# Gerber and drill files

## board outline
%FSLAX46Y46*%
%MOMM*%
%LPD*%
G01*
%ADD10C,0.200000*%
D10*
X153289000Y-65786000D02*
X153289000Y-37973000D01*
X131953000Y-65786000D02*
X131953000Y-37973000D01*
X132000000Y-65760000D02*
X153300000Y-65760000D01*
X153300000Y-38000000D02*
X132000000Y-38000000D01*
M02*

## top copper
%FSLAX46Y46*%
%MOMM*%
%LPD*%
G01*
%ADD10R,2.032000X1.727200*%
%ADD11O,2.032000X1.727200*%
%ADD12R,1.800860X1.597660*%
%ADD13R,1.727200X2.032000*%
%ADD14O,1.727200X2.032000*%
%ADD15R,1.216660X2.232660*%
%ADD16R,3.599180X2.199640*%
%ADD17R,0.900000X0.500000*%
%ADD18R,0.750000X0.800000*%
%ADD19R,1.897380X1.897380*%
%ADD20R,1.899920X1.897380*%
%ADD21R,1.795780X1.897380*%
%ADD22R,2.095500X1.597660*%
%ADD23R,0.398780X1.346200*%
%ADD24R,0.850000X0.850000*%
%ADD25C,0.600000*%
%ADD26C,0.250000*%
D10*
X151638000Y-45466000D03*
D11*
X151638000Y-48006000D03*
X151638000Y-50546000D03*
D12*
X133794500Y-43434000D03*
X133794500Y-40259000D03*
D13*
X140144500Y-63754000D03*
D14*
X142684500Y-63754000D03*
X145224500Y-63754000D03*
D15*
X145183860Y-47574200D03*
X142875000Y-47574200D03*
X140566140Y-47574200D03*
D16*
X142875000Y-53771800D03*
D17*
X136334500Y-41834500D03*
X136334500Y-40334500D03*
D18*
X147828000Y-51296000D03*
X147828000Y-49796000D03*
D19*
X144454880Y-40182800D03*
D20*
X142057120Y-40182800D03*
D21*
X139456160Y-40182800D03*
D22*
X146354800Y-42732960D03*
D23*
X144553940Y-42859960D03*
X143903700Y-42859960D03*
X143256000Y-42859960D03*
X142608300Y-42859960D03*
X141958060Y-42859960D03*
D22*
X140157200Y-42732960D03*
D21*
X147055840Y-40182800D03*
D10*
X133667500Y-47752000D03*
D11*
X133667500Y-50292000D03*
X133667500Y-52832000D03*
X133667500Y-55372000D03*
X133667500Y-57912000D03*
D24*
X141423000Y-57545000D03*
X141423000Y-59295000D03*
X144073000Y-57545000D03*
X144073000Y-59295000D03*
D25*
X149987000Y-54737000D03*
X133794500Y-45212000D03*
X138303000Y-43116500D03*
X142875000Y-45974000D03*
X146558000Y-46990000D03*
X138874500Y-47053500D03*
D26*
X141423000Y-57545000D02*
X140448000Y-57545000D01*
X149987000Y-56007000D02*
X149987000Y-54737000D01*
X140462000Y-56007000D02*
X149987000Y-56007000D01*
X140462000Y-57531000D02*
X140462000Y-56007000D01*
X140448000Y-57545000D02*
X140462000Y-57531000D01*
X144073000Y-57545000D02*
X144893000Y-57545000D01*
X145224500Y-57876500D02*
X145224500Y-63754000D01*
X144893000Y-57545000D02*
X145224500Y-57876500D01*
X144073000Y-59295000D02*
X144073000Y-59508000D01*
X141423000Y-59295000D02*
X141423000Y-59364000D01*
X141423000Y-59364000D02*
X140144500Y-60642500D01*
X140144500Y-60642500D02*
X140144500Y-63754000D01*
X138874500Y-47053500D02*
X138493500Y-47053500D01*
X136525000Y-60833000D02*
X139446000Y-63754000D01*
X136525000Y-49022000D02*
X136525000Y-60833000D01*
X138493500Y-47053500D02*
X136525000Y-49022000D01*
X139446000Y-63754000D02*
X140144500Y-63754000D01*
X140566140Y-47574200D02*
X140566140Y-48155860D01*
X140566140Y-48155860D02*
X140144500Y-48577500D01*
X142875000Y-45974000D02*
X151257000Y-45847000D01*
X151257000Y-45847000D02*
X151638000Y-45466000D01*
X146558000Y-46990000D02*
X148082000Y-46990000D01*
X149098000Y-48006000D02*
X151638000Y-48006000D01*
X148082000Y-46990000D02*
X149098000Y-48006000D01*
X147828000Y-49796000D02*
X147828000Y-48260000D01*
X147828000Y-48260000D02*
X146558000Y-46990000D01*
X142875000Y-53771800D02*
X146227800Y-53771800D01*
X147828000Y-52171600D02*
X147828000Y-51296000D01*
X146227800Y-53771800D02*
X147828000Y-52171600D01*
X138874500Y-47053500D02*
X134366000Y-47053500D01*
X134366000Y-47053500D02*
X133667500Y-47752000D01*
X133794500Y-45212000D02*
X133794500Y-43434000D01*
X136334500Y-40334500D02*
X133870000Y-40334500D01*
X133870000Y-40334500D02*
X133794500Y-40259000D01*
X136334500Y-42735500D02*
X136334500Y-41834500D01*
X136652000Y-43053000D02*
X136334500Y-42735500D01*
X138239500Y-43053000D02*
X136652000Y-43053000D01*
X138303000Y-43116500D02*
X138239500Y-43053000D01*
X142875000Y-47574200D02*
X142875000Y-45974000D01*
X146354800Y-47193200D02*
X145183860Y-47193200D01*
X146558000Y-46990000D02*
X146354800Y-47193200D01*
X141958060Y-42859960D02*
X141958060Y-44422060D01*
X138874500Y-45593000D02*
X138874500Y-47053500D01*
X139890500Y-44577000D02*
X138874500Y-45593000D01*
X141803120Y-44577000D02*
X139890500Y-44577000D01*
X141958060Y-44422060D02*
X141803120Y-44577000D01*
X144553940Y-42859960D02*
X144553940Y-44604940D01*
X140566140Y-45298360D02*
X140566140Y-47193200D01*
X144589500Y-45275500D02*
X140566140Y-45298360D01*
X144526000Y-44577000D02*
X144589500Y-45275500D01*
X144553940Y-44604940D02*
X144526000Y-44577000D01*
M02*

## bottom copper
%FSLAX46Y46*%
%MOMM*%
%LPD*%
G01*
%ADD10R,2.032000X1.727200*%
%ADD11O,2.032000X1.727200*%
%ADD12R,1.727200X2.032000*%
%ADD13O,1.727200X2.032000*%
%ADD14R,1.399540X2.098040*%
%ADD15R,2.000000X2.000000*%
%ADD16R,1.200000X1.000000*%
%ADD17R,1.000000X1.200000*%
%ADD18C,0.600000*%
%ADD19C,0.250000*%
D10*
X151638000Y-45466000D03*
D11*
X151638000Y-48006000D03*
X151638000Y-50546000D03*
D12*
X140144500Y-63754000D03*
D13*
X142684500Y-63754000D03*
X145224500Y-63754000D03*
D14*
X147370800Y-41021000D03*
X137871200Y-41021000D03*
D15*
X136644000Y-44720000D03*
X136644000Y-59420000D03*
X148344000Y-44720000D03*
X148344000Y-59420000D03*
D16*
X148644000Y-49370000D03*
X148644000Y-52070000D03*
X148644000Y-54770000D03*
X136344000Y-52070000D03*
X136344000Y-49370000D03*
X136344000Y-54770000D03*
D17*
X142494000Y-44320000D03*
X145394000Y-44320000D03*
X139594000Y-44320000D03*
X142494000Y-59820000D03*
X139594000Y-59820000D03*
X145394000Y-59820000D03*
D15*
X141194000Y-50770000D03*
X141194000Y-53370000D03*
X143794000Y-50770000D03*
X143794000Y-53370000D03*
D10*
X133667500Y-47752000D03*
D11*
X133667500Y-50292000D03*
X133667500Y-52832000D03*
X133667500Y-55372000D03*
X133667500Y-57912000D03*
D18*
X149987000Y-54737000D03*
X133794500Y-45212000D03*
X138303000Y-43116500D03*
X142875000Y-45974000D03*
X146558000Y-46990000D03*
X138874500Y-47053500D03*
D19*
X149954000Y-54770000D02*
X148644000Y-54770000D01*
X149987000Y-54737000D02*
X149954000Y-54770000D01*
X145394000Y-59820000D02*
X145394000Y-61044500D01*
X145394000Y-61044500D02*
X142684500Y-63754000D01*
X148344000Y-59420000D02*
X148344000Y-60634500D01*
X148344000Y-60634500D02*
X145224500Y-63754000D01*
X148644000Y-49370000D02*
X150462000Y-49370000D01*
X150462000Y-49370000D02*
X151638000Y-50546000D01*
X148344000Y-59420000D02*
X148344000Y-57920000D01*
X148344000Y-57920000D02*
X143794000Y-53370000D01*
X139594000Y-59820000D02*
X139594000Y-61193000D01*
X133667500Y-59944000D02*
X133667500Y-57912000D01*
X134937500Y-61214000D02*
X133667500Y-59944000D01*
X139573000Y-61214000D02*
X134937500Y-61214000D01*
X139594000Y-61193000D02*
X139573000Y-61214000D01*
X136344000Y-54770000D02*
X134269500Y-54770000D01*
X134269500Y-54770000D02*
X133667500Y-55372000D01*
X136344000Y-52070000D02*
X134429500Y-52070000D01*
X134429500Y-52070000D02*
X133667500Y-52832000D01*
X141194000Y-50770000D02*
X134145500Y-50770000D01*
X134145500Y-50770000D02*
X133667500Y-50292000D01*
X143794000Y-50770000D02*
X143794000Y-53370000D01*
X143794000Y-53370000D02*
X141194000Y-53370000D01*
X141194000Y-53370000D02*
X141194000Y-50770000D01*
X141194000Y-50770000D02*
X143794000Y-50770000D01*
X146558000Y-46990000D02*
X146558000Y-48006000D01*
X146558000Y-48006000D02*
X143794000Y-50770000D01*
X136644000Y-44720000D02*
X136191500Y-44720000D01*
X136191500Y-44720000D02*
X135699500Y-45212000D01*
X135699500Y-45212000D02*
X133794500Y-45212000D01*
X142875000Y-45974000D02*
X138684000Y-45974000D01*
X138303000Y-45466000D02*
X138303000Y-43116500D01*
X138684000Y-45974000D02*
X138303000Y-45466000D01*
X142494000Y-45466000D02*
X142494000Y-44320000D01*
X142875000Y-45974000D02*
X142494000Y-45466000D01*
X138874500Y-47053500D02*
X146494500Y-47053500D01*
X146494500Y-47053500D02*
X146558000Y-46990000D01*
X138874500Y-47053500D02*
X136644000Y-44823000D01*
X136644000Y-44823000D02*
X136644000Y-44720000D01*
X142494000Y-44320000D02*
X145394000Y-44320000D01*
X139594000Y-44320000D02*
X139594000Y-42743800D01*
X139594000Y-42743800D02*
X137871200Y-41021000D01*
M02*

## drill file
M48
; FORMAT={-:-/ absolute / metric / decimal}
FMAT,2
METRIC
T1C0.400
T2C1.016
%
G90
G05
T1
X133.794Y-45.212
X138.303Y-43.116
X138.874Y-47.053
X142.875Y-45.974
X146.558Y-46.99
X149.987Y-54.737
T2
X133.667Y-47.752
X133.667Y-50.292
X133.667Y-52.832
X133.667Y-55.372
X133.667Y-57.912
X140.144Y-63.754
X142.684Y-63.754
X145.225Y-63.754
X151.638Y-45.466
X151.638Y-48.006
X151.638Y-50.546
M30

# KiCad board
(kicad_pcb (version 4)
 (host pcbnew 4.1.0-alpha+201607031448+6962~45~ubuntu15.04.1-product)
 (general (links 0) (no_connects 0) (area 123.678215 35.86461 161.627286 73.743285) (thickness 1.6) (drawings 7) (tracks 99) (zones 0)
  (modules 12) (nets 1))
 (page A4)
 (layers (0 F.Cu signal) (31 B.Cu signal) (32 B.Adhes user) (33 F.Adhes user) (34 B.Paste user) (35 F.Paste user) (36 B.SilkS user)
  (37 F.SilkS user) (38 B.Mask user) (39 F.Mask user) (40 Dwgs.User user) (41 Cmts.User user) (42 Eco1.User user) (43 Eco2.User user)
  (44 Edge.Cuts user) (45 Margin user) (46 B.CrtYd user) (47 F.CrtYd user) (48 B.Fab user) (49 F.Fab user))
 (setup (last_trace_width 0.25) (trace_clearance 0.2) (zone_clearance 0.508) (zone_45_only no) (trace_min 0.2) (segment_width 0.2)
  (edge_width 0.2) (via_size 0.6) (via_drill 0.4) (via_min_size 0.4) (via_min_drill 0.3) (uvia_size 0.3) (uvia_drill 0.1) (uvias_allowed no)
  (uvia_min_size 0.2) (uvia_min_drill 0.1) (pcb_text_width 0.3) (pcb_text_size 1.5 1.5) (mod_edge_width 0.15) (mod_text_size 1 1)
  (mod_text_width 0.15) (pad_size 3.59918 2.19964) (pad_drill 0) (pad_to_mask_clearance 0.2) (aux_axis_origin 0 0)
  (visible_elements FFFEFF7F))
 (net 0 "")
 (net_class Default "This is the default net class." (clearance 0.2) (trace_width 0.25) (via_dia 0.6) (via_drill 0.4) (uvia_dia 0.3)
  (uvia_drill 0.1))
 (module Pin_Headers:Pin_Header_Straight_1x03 (layer F.Cu) (at 151.638 45.466)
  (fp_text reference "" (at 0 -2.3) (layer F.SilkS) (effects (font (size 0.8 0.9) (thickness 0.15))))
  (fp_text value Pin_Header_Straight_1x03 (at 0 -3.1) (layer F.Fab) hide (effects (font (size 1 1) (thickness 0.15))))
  (pad 1 thru_hole rect (at 0 0) (size 2.032 1.7272) (drill 1.016) (layers *.Cu *.Mask F.SilkS))
  (pad 2 thru_hole oval (at 0 2.54) (size 2.032 1.7272) (drill 1.016) (layers *.Cu *.Mask F.SilkS))
  (pad 3 thru_hole oval (at 0 5.08) (size 2.032 1.7272) (drill 1.016) (layers *.Cu *.Mask F.SilkS)))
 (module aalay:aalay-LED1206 (layer F.Cu) (at 133.7945 41.8465 90)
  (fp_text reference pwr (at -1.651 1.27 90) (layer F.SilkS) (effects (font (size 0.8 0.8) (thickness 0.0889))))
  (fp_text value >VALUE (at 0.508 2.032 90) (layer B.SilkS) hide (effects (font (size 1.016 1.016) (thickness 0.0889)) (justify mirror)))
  (pad A smd rect (at -1.5875 0 90) (size 1.59766 1.80086) (layers F.Cu F.Paste F.Mask))
  (pad K smd rect (at 1.5875 0 90) (size 1.59766 1.80086) (layers F.Cu F.Paste F.Mask)))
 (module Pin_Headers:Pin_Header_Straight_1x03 (layer F.Cu) (at 140.1445 63.754 90)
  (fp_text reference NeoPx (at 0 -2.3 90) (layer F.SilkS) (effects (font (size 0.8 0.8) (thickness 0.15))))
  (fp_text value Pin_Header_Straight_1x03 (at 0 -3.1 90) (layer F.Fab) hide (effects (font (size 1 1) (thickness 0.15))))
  (pad 1 thru_hole rect (at 0 0 90) (size 2.032 1.7272) (drill 1.016) (layers *.Cu *.Mask F.SilkS))
  (pad 2 thru_hole oval (at 0 2.54 90) (size 2.032 1.7272) (drill 1.016) (layers *.Cu *.Mask F.SilkS))
  (pad 3 thru_hole oval (at 0 5.08 90) (size 2.032 1.7272) (drill 1.016) (layers *.Cu *.Mask F.SilkS)))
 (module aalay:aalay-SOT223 (layer F.Cu) (at 142.875 50.673 180)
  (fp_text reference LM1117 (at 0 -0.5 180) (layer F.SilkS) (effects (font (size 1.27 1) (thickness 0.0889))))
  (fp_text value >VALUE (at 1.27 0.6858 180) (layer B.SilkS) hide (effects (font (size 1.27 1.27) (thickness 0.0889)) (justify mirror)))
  (pad GND smd rect (at -2.30886 3.0988 180) (size 1.21666 2.23266) (layers F.Cu F.Paste F.Mask))
  (pad OUT smd rect (at 0 3.0988 180) (size 1.21666 2.23266) (layers F.Cu F.Paste F.Mask))
  (pad IN smd rect (at 2.30886 3.0988 180) (size 1.21666 2.23266) (layers F.Cu F.Paste F.Mask))
  (pad OUT smd rect (at 0 -3.0988 180) (size 3.59918 2.19964) (layers F.Cu F.Paste F.Mask)))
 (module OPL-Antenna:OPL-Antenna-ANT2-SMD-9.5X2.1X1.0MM (layer B.Cu) (at 142.621 41.021 180)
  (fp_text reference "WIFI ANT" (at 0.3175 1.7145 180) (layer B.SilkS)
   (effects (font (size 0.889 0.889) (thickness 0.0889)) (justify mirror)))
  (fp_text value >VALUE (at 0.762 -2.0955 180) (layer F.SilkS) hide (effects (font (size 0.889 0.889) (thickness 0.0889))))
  (pad 1 smd rect (at -4.7498 0 180) (size 1.39954 2.09804) (layers B.Cu B.Paste B.Mask))
  (pad 2 smd rect (at 4.7498 0 180) (size 1.39954 2.09804) (layers B.Cu B.Paste B.Mask)))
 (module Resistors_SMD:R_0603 (layer F.Cu) (at 136.3345 41.0845 90)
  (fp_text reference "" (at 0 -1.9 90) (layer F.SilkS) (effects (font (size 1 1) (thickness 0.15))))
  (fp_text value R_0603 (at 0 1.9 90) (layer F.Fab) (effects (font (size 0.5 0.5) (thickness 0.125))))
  (pad 1 smd rect (at -0.75 0 90) (size 0.5 0.9) (layers F.Cu F.Paste F.Mask))
  (pad 2 smd rect (at 0.75 0 90) (size 0.5 0.9) (layers F.Cu F.Paste F.Mask)))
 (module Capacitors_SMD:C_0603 (layer F.Cu) (at 147.828 50.546 90)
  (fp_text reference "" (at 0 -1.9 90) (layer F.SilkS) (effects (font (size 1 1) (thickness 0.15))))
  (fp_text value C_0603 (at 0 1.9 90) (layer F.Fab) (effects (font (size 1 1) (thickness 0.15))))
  (pad 1 smd rect (at -0.75 0 90) (size 0.8 0.75) (layers F.Cu F.Paste F.Mask))
  (pad 2 smd rect (at 0.75 0 90) (size 0.8 0.75) (layers F.Cu F.Paste F.Mask)))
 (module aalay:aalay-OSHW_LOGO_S (layer F.Cu) (at 150.622 39.878)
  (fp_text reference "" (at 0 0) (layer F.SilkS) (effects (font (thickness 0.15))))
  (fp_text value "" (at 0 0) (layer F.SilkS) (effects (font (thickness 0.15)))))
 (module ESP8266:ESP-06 (layer B.Cu) (at 142.494 52.07 270)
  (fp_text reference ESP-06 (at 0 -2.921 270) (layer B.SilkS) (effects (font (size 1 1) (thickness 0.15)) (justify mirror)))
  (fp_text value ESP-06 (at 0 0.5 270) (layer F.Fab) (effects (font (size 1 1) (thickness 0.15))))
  (pad GND smd rect (at -7.35 5.85 270) (size 2 2) (layers B.Cu B.Paste B.Mask))
  (pad GP5 smd rect (at 7.35 5.85 270) (size 2 2) (layers B.Cu B.Paste B.Mask))
  (pad GP16 smd rect (at -7.35 -5.85 270) (size 2 2) (layers B.Cu B.Paste B.Mask))
  (pad GP15 smd rect (at 7.35 -5.85 270) (size 2 2) (layers B.Cu B.Paste B.Mask))
  (pad GP14 smd rect (at -2.7 -6.15 270) (size 1 1.2) (layers B.Cu B.Paste B.Mask))
  (pad GP12 smd rect (at 0 -6.15 270) (size 1 1.2) (layers B.Cu B.Paste B.Mask))
  (pad GP13 smd rect (at 2.7 -6.15 270) (size 1 1.2) (layers B.Cu B.Paste B.Mask))
  (pad TX smd rect (at 0 6.15 270) (size 1 1.2) (layers B.Cu B.Paste B.Mask))
  (pad RST smd rect (at -2.7 6.15 270) (size 1 1.2) (layers B.Cu B.Paste B.Mask))
  (pad RX smd rect (at 2.7 6.15 270) (size 1 1.2) (layers B.Cu B.Paste B.Mask))
  (pad 3.3 smd rect (at -7.75 0 270) (size 1.2 1) (layers B.Cu B.Paste B.Mask))
  (pad CHPD smd rect (at -7.75 -2.9 270) (size 1.2 1) (layers B.Cu B.Paste B.Mask))
  (pad ANT smd rect (at -7.75 2.9 270) (size 1.2 1) (layers B.Cu B.Paste B.Mask))
  (pad GP2 smd rect (at 7.75 0 270) (size 1.2 1) (layers B.Cu B.Paste B.Mask))
  (pad GP0 smd rect (at 7.75 2.9 270) (size 1.2 1) (layers B.Cu B.Paste B.Mask))
  (pad GP4 smd rect (at 7.75 -2.9 270) (size 1.2 1) (layers B.Cu B.Paste B.Mask))
  (pad GND smd rect (at -1.3 1.3 270) (size 2 2) (layers B.Cu B.Paste B.Mask))
  (pad GND smd rect (at 1.3 1.3 270) (size 2 2) (layers B.Cu B.Paste B.Mask))
  (pad GND smd rect (at -1.3 -1.3 270) (size 2 2) (layers B.Cu B.Paste B.Mask))
  (pad GND smd rect (at 1.3 -1.3 270) (size 2 2) (layers B.Cu B.Paste B.Mask)))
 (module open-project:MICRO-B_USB (layer F.Cu) (at 143.256 38.735 180)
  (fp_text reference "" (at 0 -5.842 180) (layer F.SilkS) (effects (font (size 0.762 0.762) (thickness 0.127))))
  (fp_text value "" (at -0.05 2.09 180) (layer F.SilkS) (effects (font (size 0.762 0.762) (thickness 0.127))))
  (pad "" smd rect (at -1.19888 -1.4478 180) (size 1.89738 1.89738) (layers F.Cu F.Paste F.Mask))
  (pad "" smd rect (at 1.19888 -1.4478 180) (size 1.89992 1.89738) (layers F.Cu F.Paste F.Mask))
  (pad "" smd rect (at 3.79984 -1.4478 180) (size 1.79578 1.89738) (layers F.Cu F.Paste F.Mask))
  (pad "" smd rect (at -3.0988 -3.99796 180) (size 2.0955 1.59766) (layers F.Cu F.Paste F.Mask))
  (pad 1 smd rect (at -1.29794 -4.12496 180) (size 0.39878 1.3462) (layers F.Cu F.Paste F.Mask) (clearance 0.2032))
  (pad 2 smd rect (at -0.6477 -4.12496 180) (size 0.39878 1.3462) (layers F.Cu F.Paste F.Mask) (clearance 0.2032))
  (pad 3 smd rect (at 0 -4.12496 180) (size 0.39878 1.3462) (layers F.Cu F.Paste F.Mask) (clearance 0.2032))
  (pad 4 smd rect (at 0.6477 -4.12496 180) (size 0.39878 1.3462) (layers F.Cu F.Paste F.Mask) (clearance 0.2032))
  (pad 5 smd rect (at 1.29794 -4.12496 180) (size 0.39878 1.3462) (layers F.Cu F.Paste F.Mask) (clearance 0.2032))
  (pad "" smd rect (at 3.0988 -3.99796 180) (size 2.0955 1.59766) (layers F.Cu F.Paste F.Mask))
  (pad "" smd rect (at -3.79984 -1.4478 180) (size 1.79578 1.89738) (layers F.Cu F.Paste F.Mask)))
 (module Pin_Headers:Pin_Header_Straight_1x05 (layer F.Cu) (at 133.6675 47.752)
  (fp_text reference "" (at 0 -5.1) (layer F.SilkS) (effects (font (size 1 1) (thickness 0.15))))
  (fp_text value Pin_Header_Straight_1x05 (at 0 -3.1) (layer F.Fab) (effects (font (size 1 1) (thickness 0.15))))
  (pad 1 thru_hole rect (at 0 0) (size 2.032 1.7272) (drill 1.016) (layers *.Cu *.Mask F.SilkS))
  (pad 2 thru_hole oval (at 0 2.54) (size 2.032 1.7272) (drill 1.016) (layers *.Cu *.Mask F.SilkS))
  (pad 3 thru_hole oval (at 0 5.08) (size 2.032 1.7272) (drill 1.016) (layers *.Cu *.Mask F.SilkS))
  (pad 4 thru_hole oval (at 0 7.62) (size 2.032 1.7272) (drill 1.016) (layers *.Cu *.Mask F.SilkS))
  (pad 5 thru_hole oval (at 0 10.16) (size 2.032 1.7272) (drill 1.016) (layers *.Cu *.Mask F.SilkS)))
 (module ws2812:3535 (layer F.Cu) (at 142.748 58.42 180)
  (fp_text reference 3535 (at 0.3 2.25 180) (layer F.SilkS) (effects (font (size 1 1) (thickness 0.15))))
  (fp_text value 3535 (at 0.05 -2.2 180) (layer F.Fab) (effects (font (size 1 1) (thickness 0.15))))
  (pad IN smd rect (at 1.325 0.875 180) (size 0.85 0.85) (layers F.Cu F.Paste F.Mask))
  (pad VDD smd rect (at 1.325 -0.875 180) (size 0.85 0.85) (layers F.Cu F.Paste F.Mask))
  (pad VSS smd rect (at -1.325 0.875 180) (size 0.85 0.85) (layers F.Cu F.Paste F.Mask))
  (pad OUT smd rect (at -1.325 -0.875 180) (size 0.85 0.85) (layers F.Cu F.Paste F.Mask)))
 (gr_line (start 153.289 65.786) (end 153.289 37.973) (angle 90) (layer Edge.Cuts) (width 0.2))
 (gr_line (start 131.953 65.786) (end 131.953 37.973) (angle 90) (layer Edge.Cuts) (width 0.2))
 (gr_line (start 132 65.76) (end 153.3 65.76) (angle 90) (layer Edge.Cuts) (width 0.2))
 (gr_line (start 153.3 38) (end 132 38) (angle 90) (layer Edge.Cuts) (width 0.2))
 (segment (start 141.423 57.545) (end 140.448 57.545) (width 0.25) (layer F.Cu) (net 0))
 (segment (start 149.954 54.77) (end 148.644 54.77) (width 0.25) (layer B.Cu) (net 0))
 (segment (start 149.987 54.737) (end 149.954 54.77) (width 0.25) (layer B.Cu) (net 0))
 (via (at 149.987 54.737) (size 0.6) (drill 0.4) (layers F.Cu B.Cu) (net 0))
 (segment (start 149.987 56.007) (end 149.987 54.737) (width 0.25) (layer F.Cu) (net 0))
 (segment (start 140.462 56.007) (end 149.987 56.007) (width 0.25) (layer F.Cu) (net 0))
 (segment (start 140.462 57.531) (end 140.462 56.007) (width 0.25) (layer F.Cu) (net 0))
 (segment (start 140.448 57.545) (end 140.462 57.531) (width 0.25) (layer F.Cu) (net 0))
 (segment (start 144.073 57.545) (end 144.893 57.545) (width 0.25) (layer F.Cu) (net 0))
 (segment (start 145.2245 57.8765) (end 145.2245 63.754) (width 0.25) (layer F.Cu) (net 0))
 (segment (start 144.893 57.545) (end 145.2245 57.8765) (width 0.25) (layer F.Cu) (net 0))
 (segment (start 144.073 59.295) (end 144.073 59.508) (width 0.25) (layer F.Cu) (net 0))
 (segment (start 141.423 59.295) (end 141.423 59.364) (width 0.25) (layer F.Cu) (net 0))
 (segment (start 141.423 59.364) (end 140.1445 60.6425) (width 0.25) (layer F.Cu) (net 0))
 (segment (start 140.1445 60.6425) (end 140.1445 63.754) (width 0.25) (layer F.Cu) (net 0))
 (segment (start 138.8745 47.0535) (end 138.4935 47.0535) (width 0.25) (layer F.Cu) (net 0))
 (segment (start 136.525 60.833) (end 139.446 63.754) (width 0.25) (layer F.Cu) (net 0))
 (segment (start 136.525 49.022) (end 136.525 60.833) (width 0.25) (layer F.Cu) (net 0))
 (segment (start 138.4935 47.0535) (end 136.525 49.022) (width 0.25) (layer F.Cu) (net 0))
 (segment (start 139.446 63.754) (end 140.1445 63.754) (width 0.25) (layer F.Cu) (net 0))
 (segment (start 140.56614 47.5742) (end 140.56614 48.15586) (width 0.25) (layer F.Cu) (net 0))
 (segment (start 140.56614 48.15586) (end 140.1445 48.5775) (width 0.25) (layer F.Cu) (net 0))
 (segment (start 145.394 59.82) (end 145.394 61.0445) (width 0.25) (layer B.Cu) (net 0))
 (segment (start 145.394 61.0445) (end 142.6845 63.754) (width 0.25) (layer B.Cu) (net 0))
 (segment (start 148.344 59.42) (end 148.344 60.6345) (width 0.25) (layer B.Cu) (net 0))
 (segment (start 148.344 60.6345) (end 145.2245 63.754) (width 0.25) (layer B.Cu) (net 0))
 (segment (start 148.644 49.37) (end 150.462 49.37) (width 0.25) (layer B.Cu) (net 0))
 (segment (start 150.462 49.37) (end 151.638 50.546) (width 0.25) (layer B.Cu) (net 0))
 (segment (start 142.875 45.974) (end 151.257 45.847) (width 0.25) (layer F.Cu) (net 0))
 (segment (start 151.257 45.847) (end 151.638 45.466) (width 0.25) (layer F.Cu) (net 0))
 (segment (start 146.558 46.99) (end 148.082 46.99) (width 0.25) (layer F.Cu) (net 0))
 (segment (start 149.098 48.006) (end 151.638 48.006) (width 0.25) (layer F.Cu) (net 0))
 (segment (start 148.082 46.99) (end 149.098 48.006) (width 0.25) (layer F.Cu) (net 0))
 (segment (start 147.828 49.796) (end 147.828 48.26) (width 0.25) (layer F.Cu) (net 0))
 (segment (start 147.828 48.26) (end 146.558 46.99) (width 0.25) (layer F.Cu) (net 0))
 (segment (start 142.875 53.7718) (end 146.2278 53.7718) (width 0.25) (layer F.Cu) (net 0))
 (segment (start 147.828 52.1716) (end 147.828 51.296) (width 0.25) (layer F.Cu) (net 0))
 (segment (start 146.2278 53.7718) (end 147.828 52.1716) (width 0.25) (layer F.Cu) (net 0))
 (segment (start 148.344 59.42) (end 148.344 57.92) (width 0.25) (layer B.Cu) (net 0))
 (segment (start 148.344 57.92) (end 143.794 53.37) (width 0.25) (layer B.Cu) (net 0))
 (segment (start 139.594 59.82) (end 139.594 61.193) (width 0.25) (layer B.Cu) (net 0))
 (segment (start 133.6675 59.944) (end 133.6675 57.912) (width 0.25) (layer B.Cu) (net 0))
 (segment (start 134.9375 61.214) (end 133.6675 59.944) (width 0.25) (layer B.Cu) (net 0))
 (segment (start 139.573 61.214) (end 134.9375 61.214) (width 0.25) (layer B.Cu) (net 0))
 (segment (start 139.594 61.193) (end 139.573 61.214) (width 0.25) (layer B.Cu) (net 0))
 (segment (start 136.344 54.77) (end 134.2695 54.77) (width 0.25) (layer B.Cu) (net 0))
 (segment (start 134.2695 54.77) (end 133.6675 55.372) (width 0.25) (layer B.Cu) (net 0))
 (segment (start 136.344 52.07) (end 134.4295 52.07) (width 0.25) (layer B.Cu) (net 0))
 (segment (start 134.4295 52.07) (end 133.6675 52.832) (width 0.25) (layer B.Cu) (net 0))
 (segment (start 141.194 50.77) (end 134.1455 50.77) (width 0.25) (layer B.Cu) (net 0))
 (segment (start 134.1455 50.77) (end 133.6675 50.292) (width 0.25) (layer B.Cu) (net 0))
 (segment (start 138.8745 47.0535) (end 134.366 47.0535) (width 0.25) (layer F.Cu) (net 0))
 (segment (start 134.366 47.0535) (end 133.6675 47.752) (width 0.25) (layer F.Cu) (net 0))
 (segment (start 143.794 50.77) (end 143.794 53.37) (width 0.25) (layer B.Cu) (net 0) (status 30))
 (segment (start 143.794 53.37) (end 141.194 53.37) (width 0.25) (layer B.Cu) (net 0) (status 30))
 (segment (start 141.194 53.37) (end 141.194 50.77) (width 0.25) (layer B.Cu) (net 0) (status 30))
 (segment (start 141.194 50.77) (end 143.794 50.77) (width 0.25) (layer B.Cu) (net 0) (status 30))
 (segment (start 146.558 46.99) (end 146.558 48.006) (width 0.25) (layer B.Cu) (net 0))
 (segment (start 146.558 48.006) (end 143.794 50.77) (width 0.25) (layer B.Cu) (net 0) (status 20))
 (segment (start 136.644 44.72) (end 136.1915 44.72) (width 0.25) (layer B.Cu) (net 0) (status 30))
 (segment (start 136.1915 44.72) (end 135.6995 45.212) (width 0.25) (layer B.Cu) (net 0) (status 30))
 (segment (start 135.6995 45.212) (end 133.7945 45.212) (width 0.25) (layer B.Cu) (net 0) (status 10))
 (via (at 133.7945 45.212) (size 0.6) (drill 0.4) (layers F.Cu B.Cu) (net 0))
 (segment (start 133.7945 45.212) (end 133.7945 43.434) (width 0.25) (layer F.Cu) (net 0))
 (segment (start 136.3345 40.3345) (end 133.87 40.3345) (width 0.25) (layer F.Cu) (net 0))
 (segment (start 133.87 40.3345) (end 133.7945 40.259) (width 0.25) (layer F.Cu) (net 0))
 (segment (start 142.875 45.974) (end 138.684 45.974) (width 0.25) (layer B.Cu) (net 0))
 (segment (start 136.3345 42.7355) (end 136.3345 41.8345) (width 0.25) (layer F.Cu) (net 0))
 (segment (start 136.652 43.053) (end 136.3345 42.7355) (width 0.25) (layer F.Cu) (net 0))
 (segment (start 138.2395 43.053) (end 136.652 43.053) (width 0.25) (layer F.Cu) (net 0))
 (segment (start 138.303 43.1165) (end 138.2395 43.053) (width 0.25) (layer F.Cu) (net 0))
 (via (at 138.303 43.1165) (size 0.6) (drill 0.4) (layers F.Cu B.Cu) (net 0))
 (segment (start 138.303 45.466) (end 138.303 43.1165) (width 0.25) (layer B.Cu) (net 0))
 (segment (start 138.684 45.974) (end 138.303 45.466) (width 0.25) (layer B.Cu) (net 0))
 (segment (start 142.875 47.5742) (end 142.875 45.974) (width 0.25) (layer F.Cu) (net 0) (status 10))
 (segment (start 142.494 45.466) (end 142.494 44.32) (width 0.25) (layer B.Cu) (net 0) (status 20))
 (segment (start 142.875 45.974) (end 142.494 45.466) (width 0.25) (layer B.Cu) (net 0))
 (via (at 142.875 45.974) (size 0.6) (drill 0.4) (layers F.Cu B.Cu) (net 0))
 (segment (start 138.8745 47.0535) (end 146.4945 47.0535) (width 0.25) (layer B.Cu) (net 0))
 (segment (start 146.3548 47.1932) (end 145.18386 47.1932) (width 0.25) (layer F.Cu) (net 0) (status 20))
 (segment (start 146.558 46.99) (end 146.3548 47.1932) (width 0.25) (layer F.Cu) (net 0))
 (via (at 146.558 46.99) (size 0.6) (drill 0.4) (layers F.Cu B.Cu) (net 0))
 (segment (start 146.4945 47.0535) (end 146.558 46.99) (width 0.25) (layer B.Cu) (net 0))
 (segment (start 141.95806 42.85996) (end 141.95806 44.42206) (width 0.25) (layer F.Cu) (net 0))
 (segment (start 138.8745 47.0535) (end 136.644 44.823) (width 0.25) (layer B.Cu) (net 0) (status 20))
 (via (at 138.8745 47.0535) (size 0.6) (drill 0.4) (layers F.Cu B.Cu) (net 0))
 (segment (start 138.8745 45.593) (end 138.8745 47.0535) (width 0.25) (layer F.Cu) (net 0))
 (segment (start 139.8905 44.577) (end 138.8745 45.593) (width 0.25) (layer F.Cu) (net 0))
 (segment (start 141.80312 44.577) (end 139.8905 44.577) (width 0.25) (layer F.Cu) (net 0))
 (segment (start 141.95806 44.42206) (end 141.80312 44.577) (width 0.25) (layer F.Cu) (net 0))
 (segment (start 136.644 44.823) (end 136.644 44.72) (width 0.25) (layer B.Cu) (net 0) (status 30))
 (segment (start 144.55394 42.85996) (end 144.55394 44.60494) (width 0.25) (layer F.Cu) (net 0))
 (segment (start 140.56614 45.29836) (end 140.56614 47.1932) (width 0.25) (layer F.Cu) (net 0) (status 20))
 (segment (start 144.5895 45.2755) (end 140.56614 45.29836) (width 0.25) (layer F.Cu) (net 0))
 (segment (start 144.526 44.577) (end 144.5895 45.2755) (width 0.25) (layer F.Cu) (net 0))
 (segment (start 144.55394 44.60494) (end 144.526 44.577) (width 0.25) (layer F.Cu) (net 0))
 (segment (start 142.494 44.32) (end 145.394 44.32) (width 0.25) (layer B.Cu) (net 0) (status 30))
 (segment (start 139.594 44.32) (end 139.594 42.7438) (width 0.25) (layer B.Cu) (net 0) (status 10))
 (segment (start 139.594 42.7438) (end 137.8712 41.021) (width 0.25) (layer B.Cu) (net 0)))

